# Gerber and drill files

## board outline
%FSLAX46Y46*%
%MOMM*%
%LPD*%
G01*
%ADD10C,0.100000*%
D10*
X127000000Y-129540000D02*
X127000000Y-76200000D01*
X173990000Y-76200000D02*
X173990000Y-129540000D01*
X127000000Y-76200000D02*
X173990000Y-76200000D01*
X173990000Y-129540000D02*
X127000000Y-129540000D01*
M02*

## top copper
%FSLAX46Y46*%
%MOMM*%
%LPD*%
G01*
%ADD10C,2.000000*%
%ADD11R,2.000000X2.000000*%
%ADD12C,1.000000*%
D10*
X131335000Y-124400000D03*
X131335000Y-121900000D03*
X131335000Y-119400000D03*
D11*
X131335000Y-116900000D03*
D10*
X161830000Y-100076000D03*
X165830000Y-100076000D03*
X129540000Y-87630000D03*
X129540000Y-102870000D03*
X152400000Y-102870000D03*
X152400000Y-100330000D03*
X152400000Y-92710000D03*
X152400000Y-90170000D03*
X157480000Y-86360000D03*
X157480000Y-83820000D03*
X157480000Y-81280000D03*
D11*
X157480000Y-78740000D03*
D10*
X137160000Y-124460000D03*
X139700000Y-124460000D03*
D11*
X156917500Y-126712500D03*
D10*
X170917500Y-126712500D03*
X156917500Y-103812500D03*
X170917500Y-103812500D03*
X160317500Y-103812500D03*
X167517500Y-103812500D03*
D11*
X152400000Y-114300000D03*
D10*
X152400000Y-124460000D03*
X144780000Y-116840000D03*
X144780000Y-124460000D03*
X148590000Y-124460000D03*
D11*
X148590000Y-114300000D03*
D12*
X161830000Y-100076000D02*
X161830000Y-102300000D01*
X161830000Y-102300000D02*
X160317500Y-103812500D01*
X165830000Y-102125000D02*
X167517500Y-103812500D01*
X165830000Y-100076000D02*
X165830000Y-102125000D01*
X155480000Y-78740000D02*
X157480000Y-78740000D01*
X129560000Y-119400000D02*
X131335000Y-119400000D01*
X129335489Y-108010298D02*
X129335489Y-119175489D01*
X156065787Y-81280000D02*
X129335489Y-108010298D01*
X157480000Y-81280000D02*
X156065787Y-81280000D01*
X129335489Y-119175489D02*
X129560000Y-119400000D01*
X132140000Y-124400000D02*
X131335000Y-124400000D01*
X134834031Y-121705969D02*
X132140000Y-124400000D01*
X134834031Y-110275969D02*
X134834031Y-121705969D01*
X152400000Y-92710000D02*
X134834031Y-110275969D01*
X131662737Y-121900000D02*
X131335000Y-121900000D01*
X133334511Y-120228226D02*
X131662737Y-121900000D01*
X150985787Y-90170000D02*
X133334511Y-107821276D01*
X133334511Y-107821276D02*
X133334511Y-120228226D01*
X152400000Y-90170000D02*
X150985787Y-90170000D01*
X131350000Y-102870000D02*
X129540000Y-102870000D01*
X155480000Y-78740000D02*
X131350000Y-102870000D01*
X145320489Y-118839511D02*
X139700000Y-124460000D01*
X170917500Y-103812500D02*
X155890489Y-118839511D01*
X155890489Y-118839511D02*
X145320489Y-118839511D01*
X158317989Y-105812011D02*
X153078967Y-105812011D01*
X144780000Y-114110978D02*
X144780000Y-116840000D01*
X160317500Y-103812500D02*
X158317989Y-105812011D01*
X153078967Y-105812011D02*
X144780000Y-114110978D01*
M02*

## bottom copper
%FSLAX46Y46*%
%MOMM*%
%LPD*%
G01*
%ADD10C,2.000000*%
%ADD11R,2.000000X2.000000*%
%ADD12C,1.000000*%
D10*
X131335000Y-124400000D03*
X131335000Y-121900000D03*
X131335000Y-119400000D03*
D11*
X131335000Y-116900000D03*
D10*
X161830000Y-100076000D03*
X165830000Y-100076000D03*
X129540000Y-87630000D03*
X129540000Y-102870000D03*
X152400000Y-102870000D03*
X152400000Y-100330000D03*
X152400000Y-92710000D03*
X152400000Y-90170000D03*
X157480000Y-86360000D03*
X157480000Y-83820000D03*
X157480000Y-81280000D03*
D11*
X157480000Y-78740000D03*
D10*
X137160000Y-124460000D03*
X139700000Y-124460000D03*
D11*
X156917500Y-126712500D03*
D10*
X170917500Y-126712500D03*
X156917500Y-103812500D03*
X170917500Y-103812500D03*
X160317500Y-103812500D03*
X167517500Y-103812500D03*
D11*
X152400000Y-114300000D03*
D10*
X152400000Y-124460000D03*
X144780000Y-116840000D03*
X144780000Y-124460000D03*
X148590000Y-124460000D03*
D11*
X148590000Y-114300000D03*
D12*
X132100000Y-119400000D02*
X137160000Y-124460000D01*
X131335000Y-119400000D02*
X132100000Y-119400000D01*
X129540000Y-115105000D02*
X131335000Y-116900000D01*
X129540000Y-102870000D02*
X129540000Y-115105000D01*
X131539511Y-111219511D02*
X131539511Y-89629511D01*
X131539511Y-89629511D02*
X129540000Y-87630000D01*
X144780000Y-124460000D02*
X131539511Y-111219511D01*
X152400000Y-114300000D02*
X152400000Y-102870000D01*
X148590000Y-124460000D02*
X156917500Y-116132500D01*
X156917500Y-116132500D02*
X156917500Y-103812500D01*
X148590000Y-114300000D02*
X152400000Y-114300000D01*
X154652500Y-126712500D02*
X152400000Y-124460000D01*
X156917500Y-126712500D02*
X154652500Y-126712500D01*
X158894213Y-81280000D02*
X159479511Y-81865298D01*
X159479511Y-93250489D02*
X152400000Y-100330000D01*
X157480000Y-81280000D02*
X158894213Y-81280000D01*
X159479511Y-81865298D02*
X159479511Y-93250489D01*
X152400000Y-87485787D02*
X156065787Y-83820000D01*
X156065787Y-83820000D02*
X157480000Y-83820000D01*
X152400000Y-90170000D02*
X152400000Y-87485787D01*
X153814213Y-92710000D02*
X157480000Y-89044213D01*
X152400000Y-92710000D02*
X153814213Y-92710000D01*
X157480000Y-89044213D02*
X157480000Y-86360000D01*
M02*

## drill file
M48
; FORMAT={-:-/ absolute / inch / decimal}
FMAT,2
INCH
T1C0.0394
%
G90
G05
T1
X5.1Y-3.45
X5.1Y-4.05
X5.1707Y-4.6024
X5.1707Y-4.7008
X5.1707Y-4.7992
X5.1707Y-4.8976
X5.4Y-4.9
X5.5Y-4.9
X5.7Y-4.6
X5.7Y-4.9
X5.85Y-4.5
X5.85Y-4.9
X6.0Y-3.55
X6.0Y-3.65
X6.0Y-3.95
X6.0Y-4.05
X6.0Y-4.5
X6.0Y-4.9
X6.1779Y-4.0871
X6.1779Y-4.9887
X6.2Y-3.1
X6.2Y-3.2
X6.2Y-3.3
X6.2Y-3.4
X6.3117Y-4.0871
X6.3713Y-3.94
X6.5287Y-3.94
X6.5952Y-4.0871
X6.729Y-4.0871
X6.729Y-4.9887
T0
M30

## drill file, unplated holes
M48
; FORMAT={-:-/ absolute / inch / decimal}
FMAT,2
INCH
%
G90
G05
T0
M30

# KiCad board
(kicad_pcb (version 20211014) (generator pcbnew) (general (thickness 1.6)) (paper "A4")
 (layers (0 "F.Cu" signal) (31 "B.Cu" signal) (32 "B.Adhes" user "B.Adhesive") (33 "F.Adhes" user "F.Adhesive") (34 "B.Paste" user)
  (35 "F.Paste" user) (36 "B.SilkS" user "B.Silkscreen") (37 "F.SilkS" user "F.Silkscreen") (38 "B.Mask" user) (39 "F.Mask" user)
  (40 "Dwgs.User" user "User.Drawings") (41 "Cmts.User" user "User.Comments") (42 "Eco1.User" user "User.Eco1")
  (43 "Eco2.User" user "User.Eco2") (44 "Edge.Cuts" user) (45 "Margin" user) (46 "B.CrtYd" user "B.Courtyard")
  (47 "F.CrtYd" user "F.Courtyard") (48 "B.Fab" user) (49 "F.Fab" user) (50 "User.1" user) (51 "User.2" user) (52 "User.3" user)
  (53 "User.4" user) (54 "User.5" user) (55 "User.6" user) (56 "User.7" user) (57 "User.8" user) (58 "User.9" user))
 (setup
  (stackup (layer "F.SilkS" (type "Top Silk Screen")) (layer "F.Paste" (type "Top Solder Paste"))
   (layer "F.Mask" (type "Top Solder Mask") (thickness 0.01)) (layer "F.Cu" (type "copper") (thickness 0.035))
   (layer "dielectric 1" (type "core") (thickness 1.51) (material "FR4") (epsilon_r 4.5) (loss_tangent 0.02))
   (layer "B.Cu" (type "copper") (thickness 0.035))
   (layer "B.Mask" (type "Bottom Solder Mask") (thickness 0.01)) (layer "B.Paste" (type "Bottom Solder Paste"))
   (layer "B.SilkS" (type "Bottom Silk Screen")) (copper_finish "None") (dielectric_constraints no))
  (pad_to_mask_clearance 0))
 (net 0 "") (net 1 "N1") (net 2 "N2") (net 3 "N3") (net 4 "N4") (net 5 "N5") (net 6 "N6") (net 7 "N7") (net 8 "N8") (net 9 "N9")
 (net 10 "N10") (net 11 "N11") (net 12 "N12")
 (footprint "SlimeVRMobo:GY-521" (layer "F.Cu") (at 163.83 87.63 -90)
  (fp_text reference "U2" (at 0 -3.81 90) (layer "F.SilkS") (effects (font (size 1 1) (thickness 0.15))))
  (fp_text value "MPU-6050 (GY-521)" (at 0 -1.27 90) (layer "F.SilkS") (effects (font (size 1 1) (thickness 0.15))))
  (pad "1" thru_hole rect (at -8.89 6.35 270) (size 2 2) (drill 1) (layers *.Cu *.Mask) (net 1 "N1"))
  (pad "2" thru_hole circle (at -6.35 6.35 270) (size 2 2) (drill 1) (layers *.Cu *.Mask) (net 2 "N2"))
  (pad "3" thru_hole circle (at -3.81 6.35 270) (size 2 2) (drill 1) (layers *.Cu *.Mask) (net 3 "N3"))
  (pad "4" thru_hole circle (at -1.27 6.35 270) (size 2 2) (drill 1) (layers *.Cu *.Mask) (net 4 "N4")))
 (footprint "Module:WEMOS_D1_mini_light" (layer "F.Cu") (at 129.54 85.09)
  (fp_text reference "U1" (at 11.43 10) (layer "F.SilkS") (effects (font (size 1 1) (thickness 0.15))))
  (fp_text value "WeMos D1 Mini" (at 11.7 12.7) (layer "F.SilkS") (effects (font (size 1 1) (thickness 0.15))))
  (pad "2" thru_hole circle (at 0 2.54) (size 2 2) (drill 1) (layers *.Cu *.Mask) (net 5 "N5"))
  (pad "8" thru_hole circle (at 0 17.78) (size 2 2) (drill 1) (layers *.Cu *.Mask) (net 1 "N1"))
  (pad "9" thru_hole circle (at 22.86 17.78) (size 2 2) (drill 1) (layers *.Cu *.Mask) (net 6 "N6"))
  (pad "10" thru_hole circle (at 22.86 15.24) (size 2 2) (drill 1) (layers *.Cu *.Mask) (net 2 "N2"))
  (pad "13" thru_hole circle (at 22.86 7.62) (size 2 2) (drill 1) (layers *.Cu *.Mask) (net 4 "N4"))
  (pad "14" thru_hole circle (at 22.86 5.08) (size 2 2) (drill 1) (layers *.Cu *.Mask) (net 3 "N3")))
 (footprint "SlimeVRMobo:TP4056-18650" (layer "F.Cu") (at 155.1175 128.4125 90)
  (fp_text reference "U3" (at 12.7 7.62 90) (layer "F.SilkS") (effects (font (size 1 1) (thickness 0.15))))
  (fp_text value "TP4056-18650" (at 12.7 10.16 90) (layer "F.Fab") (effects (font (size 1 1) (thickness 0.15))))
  (pad "1" thru_hole rect (at 1.7 1.8 90) (size 2 2) (drill 1) (layers *.Cu *.Mask) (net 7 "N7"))
  (pad "2" thru_hole circle (at 1.7 15.8 90) (size 2 2) (drill 1) (layers *.Cu *.Mask) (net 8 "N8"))
  (pad "3" thru_hole circle (at 24.6 1.8 90) (size 2 2) (drill 1) (layers *.Cu *.Mask) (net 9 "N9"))
  (pad "4" thru_hole circle (at 24.6 15.8 90) (size 2 2) (drill 1) (layers *.Cu *.Mask) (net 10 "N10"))
  (pad "5" thru_hole circle (at 24.6 5.2 90) (size 2 2) (drill 1) (layers *.Cu *.Mask) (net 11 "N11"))
  (pad "6" thru_hole circle (at 24.6 12.4 90) (size 2 2) (drill 1) (layers *.Cu *.Mask) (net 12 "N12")))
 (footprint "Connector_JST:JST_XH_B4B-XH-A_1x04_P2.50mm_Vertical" (layer "F.Cu") (at 131.335 116.9 -90)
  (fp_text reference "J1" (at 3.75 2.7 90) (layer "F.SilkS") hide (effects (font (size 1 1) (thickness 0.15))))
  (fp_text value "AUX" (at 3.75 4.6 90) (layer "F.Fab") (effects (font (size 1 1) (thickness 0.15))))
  (pad "1" thru_hole rect (at 0 0 270) (size 2 2) (drill 1) (layers *.Cu *.Mask) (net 1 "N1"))
  (pad "2" thru_hole circle (at 2.5 0 270) (size 2 2) (drill 1) (layers *.Cu *.Mask) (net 2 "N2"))
  (pad "3" thru_hole circle (at 5 0 270) (size 2 2) (drill 1) (layers *.Cu *.Mask) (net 3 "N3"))
  (pad "4" thru_hole circle (at 7.5 0 270) (size 2 2) (drill 1) (layers *.Cu *.Mask) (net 4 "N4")))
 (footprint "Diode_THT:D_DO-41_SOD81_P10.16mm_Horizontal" (layer "F.Cu") (at 152.4 114.3 -90)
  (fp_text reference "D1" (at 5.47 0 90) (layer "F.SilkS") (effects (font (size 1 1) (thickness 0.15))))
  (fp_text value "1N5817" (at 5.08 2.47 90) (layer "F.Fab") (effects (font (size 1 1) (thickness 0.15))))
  (pad "1" thru_hole rect (at 0 0 270) (size 2 2) (drill 1) (layers *.Cu *.Mask) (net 6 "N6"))
  (pad "2" thru_hole circle (at 10.16 0 270) (size 2 2) (drill 1) (layers *.Cu *.Mask) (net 7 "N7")))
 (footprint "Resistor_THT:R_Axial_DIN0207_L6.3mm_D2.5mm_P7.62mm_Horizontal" (layer "F.Cu") (at 144.78 116.84 -90)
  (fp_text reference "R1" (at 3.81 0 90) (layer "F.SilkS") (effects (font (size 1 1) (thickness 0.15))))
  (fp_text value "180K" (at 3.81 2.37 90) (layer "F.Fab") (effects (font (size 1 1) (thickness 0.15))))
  (pad "1" thru_hole circle (at 0 0 270) (size 2 2) (drill 1) (layers *.Cu *.Mask) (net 11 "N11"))
  (pad "2" thru_hole circle (at 7.62 0 270) (size 2 2) (drill 1) (layers *.Cu *.Mask) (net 5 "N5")))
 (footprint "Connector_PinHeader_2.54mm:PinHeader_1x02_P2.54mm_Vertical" (layer "F.Cu") (at 139.7 124.46 -90)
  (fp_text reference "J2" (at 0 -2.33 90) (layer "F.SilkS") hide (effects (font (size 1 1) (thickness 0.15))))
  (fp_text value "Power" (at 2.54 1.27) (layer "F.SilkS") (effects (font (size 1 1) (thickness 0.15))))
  (pad "1" thru_hole circle (at 0 0 270) (size 2 2) (drill 1) (layers *.Cu *.Mask) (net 10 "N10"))
  (pad "2" thru_hole circle (at 0 2.54 270) (size 2 2) (drill 1) (layers *.Cu *.Mask) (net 2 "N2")))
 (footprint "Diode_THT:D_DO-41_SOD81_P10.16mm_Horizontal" (layer "F.Cu") (at 148.59 114.3 -90)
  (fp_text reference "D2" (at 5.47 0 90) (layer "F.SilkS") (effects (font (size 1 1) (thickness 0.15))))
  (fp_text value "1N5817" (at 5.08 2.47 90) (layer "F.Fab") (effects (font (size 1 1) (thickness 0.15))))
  (pad "1" thru_hole rect (at 0 0 270) (size 2 2) (drill 1) (layers *.Cu *.Mask) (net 6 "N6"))
  (pad "2" thru_hole circle (at 10.16 0 270) (size 2 2) (drill 1) (layers *.Cu *.Mask) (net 9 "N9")))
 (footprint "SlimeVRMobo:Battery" (layer "F.Cu") (at 163.83 100.076 90)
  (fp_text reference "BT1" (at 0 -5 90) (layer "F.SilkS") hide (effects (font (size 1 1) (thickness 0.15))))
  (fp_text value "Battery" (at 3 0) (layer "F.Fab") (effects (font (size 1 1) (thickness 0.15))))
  (pad "1" thru_hole circle (at 0 -2 90) (size 2 2) (drill 1) (layers *.Cu *.Mask) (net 11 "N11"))
  (pad "2" thru_hole circle (at 0 2 90) (size 2 2) (drill 1) (layers *.Cu *.Mask) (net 12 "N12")))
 (gr_line (start 127 129.54) (end 127 76.2) (layer "Edge.Cuts") (width 0.1))
 (gr_line (start 173.99 76.2) (end 173.99 129.54) (layer "Edge.Cuts") (width 0.1))
 (gr_line (start 127 76.2) (end 173.99 76.2) (layer "Edge.Cuts") (width 0.1))
 (gr_line (start 173.99 129.54) (end 127 129.54) (layer "Edge.Cuts") (width 0.1))
 (segment (start 158.317989 105.812011) (end 153.078967 105.812011) (width 1) (layer "F.Cu") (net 11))
 (segment (start 153.078967 105.812011) (end 144.78 114.110978) (width 1) (layer "F.Cu") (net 11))
 (segment (start 161.83 100.076) (end 161.83 102.3) (width 1) (layer "F.Cu") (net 11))
 (segment (start 161.83 102.3) (end 160.3175 103.8125) (width 1) (layer "F.Cu") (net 11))
 (segment (start 144.78 114.110978) (end 144.78 116.84) (width 1) (layer "F.Cu") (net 11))
 (segment (start 160.3175 103.8125) (end 158.317989 105.812011) (width 1) (layer "F.Cu") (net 11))
 (segment (start 155.48 78.74) (end 157.48 78.74) (width 1) (layer "F.Cu") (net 1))
 (segment (start 131.35 102.87) (end 129.54 102.87) (width 1) (layer "F.Cu") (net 1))
 (segment (start 155.48 78.74) (end 131.35 102.87) (width 1) (layer "F.Cu") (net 1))
 (segment (start 129.54 115.105) (end 131.335 116.9) (width 1) (layer "B.Cu") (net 1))
 (segment (start 129.54 102.87) (end 129.54 115.105) (width 1) (layer "B.Cu") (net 1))
 (segment (start 148.59 114.3) (end 152.4 114.3) (width 1) (layer "B.Cu") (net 6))
 (segment (start 152.4 114.3) (end 152.4 102.87) (width 1) (layer "B.Cu") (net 6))
 (segment (start 144.78 124.46) (end 131.539511 111.219511) (width 1) (layer "B.Cu") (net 5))
 (segment (start 131.539511 89.629511) (end 129.54 87.63) (width 1) (layer "B.Cu") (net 5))
 (segment (start 131.539511 111.219511) (end 131.539511 89.629511) (width 1) (layer "B.Cu") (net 5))
 (segment (start 129.335489 108.010298) (end 129.335489 119.175489) (width 1) (layer "F.Cu") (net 2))
 (segment (start 129.335489 119.175489) (end 129.56 119.4) (width 1) (layer "F.Cu") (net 2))
 (segment (start 129.56 119.4) (end 131.335 119.4) (width 1) (layer "F.Cu") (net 2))
 (segment (start 156.065787 81.28) (end 129.335489 108.010298) (width 1) (layer "F.Cu") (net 2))
 (segment (start 157.48 81.28) (end 156.065787 81.28) (width 1) (layer "F.Cu") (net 2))
 (segment (start 158.894213 81.28) (end 159.479511 81.865298) (width 1) (layer "B.Cu") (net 2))
 (segment (start 131.335 119.4) (end 132.1 119.4) (width 1) (layer "B.Cu") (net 2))
 (segment (start 159.479511 81.865298) (end 159.479511 93.250489) (width 1) (layer "B.Cu") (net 2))
 (segment (start 132.1 119.4) (end 137.16 124.46) (width 1) (layer "B.Cu") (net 2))
 (segment (start 159.479511 93.250489) (end 152.4 100.33) (width 1) (layer "B.Cu") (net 2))
 (segment (start 157.48 81.28) (end 158.894213 81.28) (width 1) (layer "B.Cu") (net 2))
 (segment (start 165.83 102.125) (end 167.5175 103.8125) (width 1) (layer "F.Cu") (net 12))
 (segment (start 165.83 100.076) (end 165.83 102.125) (width 1) (layer "F.Cu") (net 12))
 (segment (start 156.9175 126.7125) (end 154.6525 126.7125) (width 1) (layer "B.Cu") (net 7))
 (segment (start 154.6525 126.7125) (end 152.4 124.46) (width 1) (layer "B.Cu") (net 7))
 (segment (start 148.59 124.46) (end 156.9175 116.1325) (width 1) (layer "B.Cu") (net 9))
 (segment (start 156.9175 116.1325) (end 156.9175 103.8125) (width 1) (layer "B.Cu") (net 9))
 (segment (start 145.320489 118.839511) (end 139.7 124.46) (width 1) (layer "F.Cu") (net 10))
 (segment (start 170.9175 103.8125) (end 155.890489 118.839511) (width 1) (layer "F.Cu") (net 10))
 (segment (start 155.890489 118.839511) (end 145.320489 118.839511) (width 1) (layer "F.Cu") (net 10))
 (segment (start 134.834031 110.275969) (end 134.834031 121.705969) (width 1) (layer "F.Cu") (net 4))
 (segment (start 132.14 124.4) (end 131.335 124.4) (width 1) (layer "F.Cu") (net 4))
 (segment (start 134.834031 121.705969) (end 132.14 124.4) (width 1) (layer "F.Cu") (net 4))
 (segment (start 152.4 92.71) (end 134.834031 110.275969) (width 1) (layer "F.Cu") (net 4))
 (segment (start 157.48 89.044213) (end 157.48 86.36) (width 1) (layer "B.Cu") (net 4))
 (segment (start 152.4 92.71) (end 153.814213 92.71) (width 1) (layer "B.Cu") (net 4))
 (segment (start 153.814213 92.71) (end 157.48 89.044213) (width 1) (layer "B.Cu") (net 4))
 (segment (start 133.334511 120.228226) (end 131.662737 121.9) (width 1) (layer "F.Cu") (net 3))
 (segment (start 133.334511 107.821276) (end 133.334511 120.228226) (width 1) (layer "F.Cu") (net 3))
 (segment (start 152.4 90.17) (end 150.985787 90.17) (width 1) (layer "F.Cu") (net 3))
 (segment (start 150.985787 90.17) (end 133.334511 107.821276) (width 1) (layer "F.Cu") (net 3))
 (segment (start 131.662737 121.9) (end 131.335 121.9) (width 1) (layer "F.Cu") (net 3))
 (segment (start 156.065787 83.82) (end 157.48 83.82) (width 1) (layer "B.Cu") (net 3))
 (segment (start 152.4 87.485787) (end 156.065787 83.82) (width 1) (layer "B.Cu") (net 3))
 (segment (start 152.4 90.17) (end 152.4 87.485787) (width 1) (layer "B.Cu") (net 3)))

